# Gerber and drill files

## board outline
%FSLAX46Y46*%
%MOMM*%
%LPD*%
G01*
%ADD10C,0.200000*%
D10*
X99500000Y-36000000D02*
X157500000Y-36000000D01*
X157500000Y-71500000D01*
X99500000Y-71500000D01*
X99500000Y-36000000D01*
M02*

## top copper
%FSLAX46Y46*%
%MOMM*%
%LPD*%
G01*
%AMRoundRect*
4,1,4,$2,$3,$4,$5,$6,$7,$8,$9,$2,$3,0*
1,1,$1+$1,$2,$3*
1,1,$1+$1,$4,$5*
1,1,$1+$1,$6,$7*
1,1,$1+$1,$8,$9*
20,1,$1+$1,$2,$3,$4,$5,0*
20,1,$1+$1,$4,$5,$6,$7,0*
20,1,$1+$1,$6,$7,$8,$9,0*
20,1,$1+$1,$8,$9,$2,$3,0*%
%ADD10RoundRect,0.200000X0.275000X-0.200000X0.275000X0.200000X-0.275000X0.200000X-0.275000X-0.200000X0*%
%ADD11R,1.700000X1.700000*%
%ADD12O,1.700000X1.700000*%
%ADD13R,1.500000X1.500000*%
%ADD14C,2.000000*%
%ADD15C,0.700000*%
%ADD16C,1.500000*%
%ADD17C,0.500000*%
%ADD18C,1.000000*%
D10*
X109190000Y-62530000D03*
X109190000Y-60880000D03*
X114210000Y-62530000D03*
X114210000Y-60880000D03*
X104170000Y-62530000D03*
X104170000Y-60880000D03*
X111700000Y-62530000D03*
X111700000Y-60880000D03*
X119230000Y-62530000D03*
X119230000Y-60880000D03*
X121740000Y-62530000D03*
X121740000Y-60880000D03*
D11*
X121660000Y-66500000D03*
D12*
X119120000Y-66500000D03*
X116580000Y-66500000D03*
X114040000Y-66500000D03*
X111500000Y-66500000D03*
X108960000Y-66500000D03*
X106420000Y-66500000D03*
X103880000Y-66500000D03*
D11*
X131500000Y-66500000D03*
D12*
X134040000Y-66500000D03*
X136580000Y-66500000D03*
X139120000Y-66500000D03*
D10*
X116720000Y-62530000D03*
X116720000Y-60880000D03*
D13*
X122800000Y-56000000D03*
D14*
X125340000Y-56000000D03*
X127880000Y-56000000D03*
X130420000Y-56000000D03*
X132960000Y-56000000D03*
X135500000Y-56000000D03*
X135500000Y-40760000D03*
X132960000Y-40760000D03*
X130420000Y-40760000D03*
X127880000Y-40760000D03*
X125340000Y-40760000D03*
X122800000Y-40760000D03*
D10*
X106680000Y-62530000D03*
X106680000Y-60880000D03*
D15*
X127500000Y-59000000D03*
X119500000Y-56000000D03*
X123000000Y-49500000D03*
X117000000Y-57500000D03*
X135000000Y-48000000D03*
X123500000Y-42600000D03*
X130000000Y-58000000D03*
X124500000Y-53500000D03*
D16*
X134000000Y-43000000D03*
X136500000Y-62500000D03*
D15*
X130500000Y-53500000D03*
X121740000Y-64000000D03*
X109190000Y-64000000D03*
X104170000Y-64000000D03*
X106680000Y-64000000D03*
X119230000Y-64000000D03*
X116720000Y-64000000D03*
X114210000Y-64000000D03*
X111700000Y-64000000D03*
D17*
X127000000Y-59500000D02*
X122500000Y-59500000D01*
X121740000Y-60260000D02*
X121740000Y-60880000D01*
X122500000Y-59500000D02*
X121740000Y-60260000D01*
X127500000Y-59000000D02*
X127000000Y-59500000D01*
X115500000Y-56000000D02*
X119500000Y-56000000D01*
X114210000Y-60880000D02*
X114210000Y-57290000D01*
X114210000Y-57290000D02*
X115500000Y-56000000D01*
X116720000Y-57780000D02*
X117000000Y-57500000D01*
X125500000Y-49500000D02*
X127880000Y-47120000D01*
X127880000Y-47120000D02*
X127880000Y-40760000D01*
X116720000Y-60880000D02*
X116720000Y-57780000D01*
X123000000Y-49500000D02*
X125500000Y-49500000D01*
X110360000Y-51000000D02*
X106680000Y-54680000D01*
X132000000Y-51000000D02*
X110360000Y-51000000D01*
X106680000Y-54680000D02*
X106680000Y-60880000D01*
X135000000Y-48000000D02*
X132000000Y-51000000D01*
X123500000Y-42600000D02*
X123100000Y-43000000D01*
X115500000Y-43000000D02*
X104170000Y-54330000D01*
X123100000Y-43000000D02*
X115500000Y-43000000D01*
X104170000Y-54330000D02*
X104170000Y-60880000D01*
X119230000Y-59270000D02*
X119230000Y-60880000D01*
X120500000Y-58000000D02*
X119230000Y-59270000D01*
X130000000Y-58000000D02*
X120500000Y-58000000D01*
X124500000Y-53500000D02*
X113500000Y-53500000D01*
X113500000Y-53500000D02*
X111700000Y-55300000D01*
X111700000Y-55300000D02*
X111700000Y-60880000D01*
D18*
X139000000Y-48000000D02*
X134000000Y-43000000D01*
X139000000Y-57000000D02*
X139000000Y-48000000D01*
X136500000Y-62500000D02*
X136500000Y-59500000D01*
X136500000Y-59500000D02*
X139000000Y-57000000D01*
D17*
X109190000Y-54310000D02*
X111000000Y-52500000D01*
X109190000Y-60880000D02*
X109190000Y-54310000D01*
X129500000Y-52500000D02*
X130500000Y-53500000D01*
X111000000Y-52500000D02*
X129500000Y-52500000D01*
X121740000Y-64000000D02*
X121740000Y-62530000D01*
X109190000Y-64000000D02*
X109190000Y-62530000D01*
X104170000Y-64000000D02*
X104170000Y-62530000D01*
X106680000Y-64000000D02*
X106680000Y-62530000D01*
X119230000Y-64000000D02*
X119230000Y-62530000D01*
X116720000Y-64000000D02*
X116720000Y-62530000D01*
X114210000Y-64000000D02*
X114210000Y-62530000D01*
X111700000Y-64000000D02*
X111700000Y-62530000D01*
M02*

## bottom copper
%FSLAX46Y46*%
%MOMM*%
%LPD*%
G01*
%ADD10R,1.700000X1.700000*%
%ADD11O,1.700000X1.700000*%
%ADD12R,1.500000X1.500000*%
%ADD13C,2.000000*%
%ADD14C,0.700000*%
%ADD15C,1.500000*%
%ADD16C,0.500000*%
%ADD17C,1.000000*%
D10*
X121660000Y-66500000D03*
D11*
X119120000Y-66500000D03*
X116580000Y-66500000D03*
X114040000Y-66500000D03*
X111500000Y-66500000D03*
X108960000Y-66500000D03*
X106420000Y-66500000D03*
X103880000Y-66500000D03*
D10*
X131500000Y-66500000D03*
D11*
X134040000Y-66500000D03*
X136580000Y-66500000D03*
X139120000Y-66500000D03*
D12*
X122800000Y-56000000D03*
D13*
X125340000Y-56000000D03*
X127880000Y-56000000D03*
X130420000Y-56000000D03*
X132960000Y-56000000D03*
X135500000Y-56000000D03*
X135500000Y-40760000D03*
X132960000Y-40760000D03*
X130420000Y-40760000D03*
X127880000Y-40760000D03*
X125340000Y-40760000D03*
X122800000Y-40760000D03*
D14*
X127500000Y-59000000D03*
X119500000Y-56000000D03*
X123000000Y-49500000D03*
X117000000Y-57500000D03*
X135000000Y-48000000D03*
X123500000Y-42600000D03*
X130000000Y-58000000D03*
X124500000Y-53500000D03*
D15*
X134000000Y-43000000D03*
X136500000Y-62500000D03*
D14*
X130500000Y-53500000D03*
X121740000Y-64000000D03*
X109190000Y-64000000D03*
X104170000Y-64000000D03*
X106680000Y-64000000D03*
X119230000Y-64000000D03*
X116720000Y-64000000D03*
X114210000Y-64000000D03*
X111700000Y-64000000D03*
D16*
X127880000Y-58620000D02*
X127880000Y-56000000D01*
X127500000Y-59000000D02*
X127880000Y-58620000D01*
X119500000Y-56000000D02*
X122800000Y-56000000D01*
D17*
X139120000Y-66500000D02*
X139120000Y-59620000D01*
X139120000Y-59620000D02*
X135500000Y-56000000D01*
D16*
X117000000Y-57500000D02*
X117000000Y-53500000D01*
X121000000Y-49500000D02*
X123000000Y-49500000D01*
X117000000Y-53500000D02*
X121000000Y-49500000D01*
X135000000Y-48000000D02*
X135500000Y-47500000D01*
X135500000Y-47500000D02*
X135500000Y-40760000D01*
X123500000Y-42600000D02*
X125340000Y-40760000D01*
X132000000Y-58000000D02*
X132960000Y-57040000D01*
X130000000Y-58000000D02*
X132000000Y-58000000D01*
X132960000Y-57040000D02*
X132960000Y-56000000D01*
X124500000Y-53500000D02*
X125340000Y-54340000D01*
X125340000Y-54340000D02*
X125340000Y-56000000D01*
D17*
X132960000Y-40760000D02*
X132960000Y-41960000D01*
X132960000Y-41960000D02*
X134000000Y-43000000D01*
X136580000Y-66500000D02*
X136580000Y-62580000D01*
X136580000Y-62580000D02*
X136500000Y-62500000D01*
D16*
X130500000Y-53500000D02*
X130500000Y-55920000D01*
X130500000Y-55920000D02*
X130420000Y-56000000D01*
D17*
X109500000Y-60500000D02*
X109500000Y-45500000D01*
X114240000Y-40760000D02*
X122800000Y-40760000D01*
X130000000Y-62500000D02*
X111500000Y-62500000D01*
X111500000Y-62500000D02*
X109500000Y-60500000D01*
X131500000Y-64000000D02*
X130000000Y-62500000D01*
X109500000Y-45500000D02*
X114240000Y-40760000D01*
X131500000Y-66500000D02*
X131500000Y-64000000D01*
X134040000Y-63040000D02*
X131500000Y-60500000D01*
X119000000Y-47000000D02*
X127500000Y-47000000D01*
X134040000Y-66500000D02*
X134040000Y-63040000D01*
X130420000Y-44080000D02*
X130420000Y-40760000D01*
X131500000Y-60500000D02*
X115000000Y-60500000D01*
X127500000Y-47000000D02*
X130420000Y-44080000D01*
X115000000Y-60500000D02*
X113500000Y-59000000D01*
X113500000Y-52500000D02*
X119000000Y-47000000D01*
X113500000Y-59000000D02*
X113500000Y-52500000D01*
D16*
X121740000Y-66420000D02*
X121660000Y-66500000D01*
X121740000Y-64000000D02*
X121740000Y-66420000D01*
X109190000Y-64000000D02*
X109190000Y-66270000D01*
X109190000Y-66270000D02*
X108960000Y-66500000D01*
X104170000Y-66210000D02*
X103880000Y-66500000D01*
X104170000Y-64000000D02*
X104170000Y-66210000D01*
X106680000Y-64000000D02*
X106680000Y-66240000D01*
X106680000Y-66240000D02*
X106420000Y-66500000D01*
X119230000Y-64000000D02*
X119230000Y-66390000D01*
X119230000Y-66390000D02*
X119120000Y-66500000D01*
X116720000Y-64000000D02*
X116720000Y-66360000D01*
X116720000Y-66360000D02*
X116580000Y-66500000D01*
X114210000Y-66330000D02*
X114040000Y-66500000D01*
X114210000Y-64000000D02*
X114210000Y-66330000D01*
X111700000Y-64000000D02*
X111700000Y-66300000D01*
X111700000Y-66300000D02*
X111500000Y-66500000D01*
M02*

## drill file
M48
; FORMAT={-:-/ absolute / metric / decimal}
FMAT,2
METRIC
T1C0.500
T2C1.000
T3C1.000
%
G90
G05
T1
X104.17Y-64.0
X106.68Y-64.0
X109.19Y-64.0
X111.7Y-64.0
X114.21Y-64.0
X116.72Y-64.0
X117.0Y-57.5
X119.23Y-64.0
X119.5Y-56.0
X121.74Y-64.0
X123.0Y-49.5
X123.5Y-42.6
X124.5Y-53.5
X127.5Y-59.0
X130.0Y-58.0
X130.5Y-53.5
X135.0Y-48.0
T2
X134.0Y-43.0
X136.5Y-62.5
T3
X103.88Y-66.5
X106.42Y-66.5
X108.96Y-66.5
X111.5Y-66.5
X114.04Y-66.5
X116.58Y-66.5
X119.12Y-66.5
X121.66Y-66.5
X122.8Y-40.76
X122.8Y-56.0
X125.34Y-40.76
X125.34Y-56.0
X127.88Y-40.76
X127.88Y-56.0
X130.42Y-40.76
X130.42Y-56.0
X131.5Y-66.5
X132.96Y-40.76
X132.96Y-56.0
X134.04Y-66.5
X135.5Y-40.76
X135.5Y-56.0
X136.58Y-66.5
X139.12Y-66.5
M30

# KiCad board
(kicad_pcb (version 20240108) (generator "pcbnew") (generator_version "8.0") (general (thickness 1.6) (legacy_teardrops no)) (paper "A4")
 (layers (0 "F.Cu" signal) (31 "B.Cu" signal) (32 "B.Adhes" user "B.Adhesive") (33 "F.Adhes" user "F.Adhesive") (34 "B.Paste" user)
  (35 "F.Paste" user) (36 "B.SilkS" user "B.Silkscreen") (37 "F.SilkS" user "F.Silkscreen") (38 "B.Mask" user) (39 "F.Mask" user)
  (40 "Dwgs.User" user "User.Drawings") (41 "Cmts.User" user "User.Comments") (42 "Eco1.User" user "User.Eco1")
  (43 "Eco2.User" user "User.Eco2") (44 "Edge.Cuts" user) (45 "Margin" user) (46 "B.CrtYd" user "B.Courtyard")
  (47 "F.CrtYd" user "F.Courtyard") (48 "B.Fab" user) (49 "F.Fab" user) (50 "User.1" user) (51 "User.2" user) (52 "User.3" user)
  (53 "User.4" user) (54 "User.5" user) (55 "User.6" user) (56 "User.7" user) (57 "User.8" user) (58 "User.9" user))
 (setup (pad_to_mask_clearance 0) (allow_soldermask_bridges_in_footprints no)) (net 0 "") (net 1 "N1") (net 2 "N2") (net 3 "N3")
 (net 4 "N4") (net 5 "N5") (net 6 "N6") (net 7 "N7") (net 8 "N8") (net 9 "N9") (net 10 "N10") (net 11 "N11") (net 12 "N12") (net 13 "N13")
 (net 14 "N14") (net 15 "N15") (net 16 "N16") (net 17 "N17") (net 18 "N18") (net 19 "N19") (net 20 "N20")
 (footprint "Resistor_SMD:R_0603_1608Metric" (layer "F.Cu") (at 109.19 61.705 90)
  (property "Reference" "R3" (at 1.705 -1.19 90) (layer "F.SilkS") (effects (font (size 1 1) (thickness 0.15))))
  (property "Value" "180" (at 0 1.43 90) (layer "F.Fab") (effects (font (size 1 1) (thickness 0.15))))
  (pad "1" smd roundrect (at -0.825 0 90) (size 0.8 0.95) (layers "F.Cu" "F.Paste" "F.Mask") (roundrect_rratio 0.25) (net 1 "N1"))
  (pad "2" smd roundrect (at 0.825 0 90) (size 0.8 0.95) (layers "F.Cu" "F.Paste" "F.Mask") (roundrect_rratio 0.25) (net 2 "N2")))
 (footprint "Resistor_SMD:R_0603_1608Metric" (layer "F.Cu") (at 114.21 61.705 90)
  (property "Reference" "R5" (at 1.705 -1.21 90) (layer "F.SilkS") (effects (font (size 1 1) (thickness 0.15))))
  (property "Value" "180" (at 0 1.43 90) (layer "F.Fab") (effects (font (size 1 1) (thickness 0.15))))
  (pad "1" smd roundrect (at -0.825 0 90) (size 0.8 0.95) (layers "F.Cu" "F.Paste" "F.Mask") (roundrect_rratio 0.25) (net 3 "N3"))
  (pad "2" smd roundrect (at 0.825 0 90) (size 0.8 0.95) (layers "F.Cu" "F.Paste" "F.Mask") (roundrect_rratio 0.25) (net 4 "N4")))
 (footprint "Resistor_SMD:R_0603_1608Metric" (layer "F.Cu") (at 104.17 61.705 90)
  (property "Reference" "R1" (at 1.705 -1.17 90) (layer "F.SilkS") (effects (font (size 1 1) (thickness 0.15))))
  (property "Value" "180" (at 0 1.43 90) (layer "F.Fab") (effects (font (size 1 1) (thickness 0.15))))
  (pad "1" smd roundrect (at -0.825 0 90) (size 0.8 0.95) (layers "F.Cu" "F.Paste" "F.Mask") (roundrect_rratio 0.25) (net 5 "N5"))
  (pad "2" smd roundrect (at 0.825 0 90) (size 0.8 0.95) (layers "F.Cu" "F.Paste" "F.Mask") (roundrect_rratio 0.25) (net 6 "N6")))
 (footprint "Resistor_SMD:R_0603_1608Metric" (layer "F.Cu") (at 111.7 61.705 90)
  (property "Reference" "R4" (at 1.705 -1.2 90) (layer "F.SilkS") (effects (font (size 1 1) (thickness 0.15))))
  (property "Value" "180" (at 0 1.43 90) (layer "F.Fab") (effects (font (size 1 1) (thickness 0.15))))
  (pad "1" smd roundrect (at -0.825 0 90) (size 0.8 0.95) (layers "F.Cu" "F.Paste" "F.Mask") (roundrect_rratio 0.25) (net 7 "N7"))
  (pad "2" smd roundrect (at 0.825 0 90) (size 0.8 0.95) (layers "F.Cu" "F.Paste" "F.Mask") (roundrect_rratio 0.25) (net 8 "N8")))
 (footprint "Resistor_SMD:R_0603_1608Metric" (layer "F.Cu") (at 119.23 61.705 90)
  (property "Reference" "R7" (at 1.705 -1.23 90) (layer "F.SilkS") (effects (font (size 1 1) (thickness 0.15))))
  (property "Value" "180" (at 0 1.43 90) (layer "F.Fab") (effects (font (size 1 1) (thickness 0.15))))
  (pad "1" smd roundrect (at -0.825 0 90) (size 0.8 0.95) (layers "F.Cu" "F.Paste" "F.Mask") (roundrect_rratio 0.25) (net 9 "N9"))
  (pad "2" smd roundrect (at 0.825 0 90) (size 0.8 0.95) (layers "F.Cu" "F.Paste" "F.Mask") (roundrect_rratio 0.25) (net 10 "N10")))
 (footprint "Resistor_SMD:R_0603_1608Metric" (layer "F.Cu") (at 121.74 61.705 90)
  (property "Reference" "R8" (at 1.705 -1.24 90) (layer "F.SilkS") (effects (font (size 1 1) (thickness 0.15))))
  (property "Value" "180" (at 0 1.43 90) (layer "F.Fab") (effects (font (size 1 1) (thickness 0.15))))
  (pad "1" smd roundrect (at -0.825 0 90) (size 0.8 0.95) (layers "F.Cu" "F.Paste" "F.Mask") (roundrect_rratio 0.25) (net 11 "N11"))
  (pad "2" smd roundrect (at 0.825 0 90) (size 0.8 0.95) (layers "F.Cu" "F.Paste" "F.Mask") (roundrect_rratio 0.25) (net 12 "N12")))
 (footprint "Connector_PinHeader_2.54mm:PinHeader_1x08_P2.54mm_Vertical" (layer "F.Cu") (at 121.66 66.5 -90)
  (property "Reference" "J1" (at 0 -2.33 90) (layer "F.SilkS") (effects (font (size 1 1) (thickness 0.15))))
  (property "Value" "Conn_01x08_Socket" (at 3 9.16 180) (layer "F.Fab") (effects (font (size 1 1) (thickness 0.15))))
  (pad "1" thru_hole rect (at 0 0 270) (size 1.7 1.7) (drill 1) (layers "*.Cu" "*.Mask") (remove_unused_layers no) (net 11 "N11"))
  (pad "2" thru_hole oval (at 0 2.54 270) (size 1.7 1.7) (drill 1) (layers "*.Cu" "*.Mask") (remove_unused_layers no) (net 9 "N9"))
  (pad "3" thru_hole oval (at 0 5.08 270) (size 1.7 1.7) (drill 1) (layers "*.Cu" "*.Mask") (remove_unused_layers no) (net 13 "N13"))
  (pad "4" thru_hole oval (at 0 7.62 270) (size 1.7 1.7) (drill 1) (layers "*.Cu" "*.Mask") (remove_unused_layers no) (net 3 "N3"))
  (pad "5" thru_hole oval (at 0 10.16 270) (size 1.7 1.7) (drill 1) (layers "*.Cu" "*.Mask") (remove_unused_layers no) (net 7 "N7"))
  (pad "6" thru_hole oval (at 0 12.7 270) (size 1.7 1.7) (drill 1) (layers "*.Cu" "*.Mask") (remove_unused_layers no) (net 1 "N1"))
  (pad "7" thru_hole oval (at 0 15.24 270) (size 1.7 1.7) (drill 1) (layers "*.Cu" "*.Mask") (remove_unused_layers no) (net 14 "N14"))
  (pad "8" thru_hole oval (at 0 17.78 270) (size 1.7 1.7) (drill 1) (layers "*.Cu" "*.Mask") (remove_unused_layers no) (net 5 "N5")))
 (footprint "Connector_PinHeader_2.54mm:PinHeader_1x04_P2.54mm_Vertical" (layer "F.Cu") (at 131.5 66.5 90)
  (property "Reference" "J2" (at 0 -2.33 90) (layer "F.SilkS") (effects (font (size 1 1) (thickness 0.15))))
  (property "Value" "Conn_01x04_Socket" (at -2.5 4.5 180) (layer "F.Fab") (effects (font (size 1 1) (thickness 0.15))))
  (pad "1" thru_hole rect (at 0 0 90) (size 1.7 1.7) (drill 1) (layers "*.Cu" "*.Mask") (remove_unused_layers no) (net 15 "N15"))
  (pad "2" thru_hole oval (at 0 2.54 90) (size 1.7 1.7) (drill 1) (layers "*.Cu" "*.Mask") (remove_unused_layers no) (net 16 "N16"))
  (pad "3" thru_hole oval (at 0 5.08 90) (size 1.7 1.7) (drill 1) (layers "*.Cu" "*.Mask") (remove_unused_layers no) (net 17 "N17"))
  (pad "4" thru_hole oval (at 0 7.62 90) (size 1.7 1.7) (drill 1) (layers "*.Cu" "*.Mask") (remove_unused_layers no) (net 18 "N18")))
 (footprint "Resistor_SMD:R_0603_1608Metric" (layer "F.Cu") (at 116.72 61.705 90)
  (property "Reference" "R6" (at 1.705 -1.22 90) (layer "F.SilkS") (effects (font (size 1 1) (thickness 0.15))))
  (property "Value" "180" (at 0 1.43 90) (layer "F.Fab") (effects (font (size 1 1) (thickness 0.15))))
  (pad "1" smd roundrect (at -0.825 0 90) (size 0.8 0.95) (layers "F.Cu" "F.Paste" "F.Mask") (roundrect_rratio 0.25) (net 13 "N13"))
  (pad "2" smd roundrect (at 0.825 0 90) (size 0.8 0.95) (layers "F.Cu" "F.Paste" "F.Mask") (roundrect_rratio 0.25) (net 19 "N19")))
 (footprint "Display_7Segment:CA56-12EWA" (layer "F.Cu") (at 122.8 56 90)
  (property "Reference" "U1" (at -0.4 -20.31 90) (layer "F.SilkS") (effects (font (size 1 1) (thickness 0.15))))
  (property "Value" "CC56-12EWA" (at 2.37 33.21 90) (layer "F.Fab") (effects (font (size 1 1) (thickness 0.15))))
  (pad "1" thru_hole rect (at 0 0 90) (size 1.5 1.5) (drill 1) (layers "*.Cu" "*.Mask") (remove_unused_layers no) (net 4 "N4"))
  (pad "2" thru_hole circle (at 0 2.54 90) (size 2 2) (drill 1) (layers "*.Cu" "*.Mask") (remove_unused_layers no) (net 8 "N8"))
  (pad "3" thru_hole circle (at 0 5.08 90) (size 2 2) (drill 1) (layers "*.Cu" "*.Mask") (remove_unused_layers no) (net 12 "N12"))
  (pad "4" thru_hole circle (at 0 7.62 90) (size 2 2) (drill 1) (layers "*.Cu" "*.Mask") (remove_unused_layers no) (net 2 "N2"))
  (pad "5" thru_hole circle (at 0 10.16 90) (size 2 2) (drill 1) (layers "*.Cu" "*.Mask") (remove_unused_layers no) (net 10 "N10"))
  (pad "6" thru_hole circle (at 0 12.7 90) (size 2 2) (drill 1) (layers "*.Cu" "*.Mask") (remove_unused_layers no) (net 18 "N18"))
  (pad "7" thru_hole circle (at 15.24 12.7 90) (size 2 2) (drill 1) (layers "*.Cu" "*.Mask") (remove_unused_layers no) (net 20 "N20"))
  (pad "8" thru_hole circle (at 15.24 10.16 90) (size 2 2) (drill 1) (layers "*.Cu" "*.Mask") (remove_unused_layers no) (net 17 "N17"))
  (pad "9" thru_hole circle (at 15.24 7.62 90) (size 2 2) (drill 1) (layers "*.Cu" "*.Mask") (remove_unused_layers no) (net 16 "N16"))
  (pad "10" thru_hole circle (at 15.24 5.08 90) (size 2 2) (drill 1) (layers "*.Cu" "*.Mask") (remove_unused_layers no) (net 19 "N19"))
  (pad "11" thru_hole circle (at 15.24 2.54 90) (size 2 2) (drill 1) (layers "*.Cu" "*.Mask") (remove_unused_layers no) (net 6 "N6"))
  (pad "12" thru_hole circle (at 15.24 0 90) (size 2 2) (drill 1) (layers "*.Cu" "*.Mask") (remove_unused_layers no) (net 15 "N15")))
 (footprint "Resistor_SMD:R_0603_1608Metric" (layer "F.Cu") (at 106.68 61.705 90)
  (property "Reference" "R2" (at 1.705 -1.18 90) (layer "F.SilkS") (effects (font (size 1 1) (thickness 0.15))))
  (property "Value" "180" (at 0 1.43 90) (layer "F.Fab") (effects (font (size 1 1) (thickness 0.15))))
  (pad "1" smd roundrect (at -0.825 0 90) (size 0.8 0.95) (layers "F.Cu" "F.Paste" "F.Mask") (roundrect_rratio 0.25) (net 14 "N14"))
  (pad "2" smd roundrect (at 0.825 0 90) (size 0.8 0.95) (layers "F.Cu" "F.Paste" "F.Mask") (roundrect_rratio 0.25) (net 20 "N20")))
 (gr_rect (start 99.5 36) (end 157.5 71.5) (stroke (width 0.2) (type default)) (fill none) (layer "Edge.Cuts"))
 (segment (start 127 59.5) (end 122.5 59.5) (width 0.5) (layer "F.Cu") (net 12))
 (segment (start 121.74 60.26) (end 121.74 60.88) (width 0.5) (layer "F.Cu") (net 12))
 (segment (start 122.5 59.5) (end 121.74 60.26) (width 0.5) (layer "F.Cu") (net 12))
 (segment (start 127.5 59) (end 127 59.5) (width 0.5) (layer "F.Cu") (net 12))
 (via (at 127.5 59) (size 0.7) (drill 0.5) (layers "F.Cu" "B.Cu") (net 12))
 (segment (start 127.88 58.62) (end 127.88 56) (width 0.5) (layer "B.Cu") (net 12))
 (segment (start 127.5 59) (end 127.88 58.62) (width 0.5) (layer "B.Cu") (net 12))
 (segment (start 115.5 56) (end 119.5 56) (width 0.5) (layer "F.Cu") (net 4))
 (segment (start 114.21 60.88) (end 114.21 57.29) (width 0.5) (layer "F.Cu") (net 4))
 (segment (start 114.21 57.29) (end 115.5 56) (width 0.5) (layer "F.Cu") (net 4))
 (via (at 119.5 56) (size 0.7) (drill 0.5) (layers "F.Cu" "B.Cu") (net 4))
 (segment (start 119.5 56) (end 122.8 56) (width 0.5) (layer "B.Cu") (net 4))
 (segment (start 139.12 66.5) (end 139.12 59.62) (width 1) (layer "B.Cu") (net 18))
 (segment (start 139.12 59.62) (end 135.5 56) (width 1) (layer "B.Cu") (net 18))
 (segment (start 116.72 57.78) (end 117 57.5) (width 0.5) (layer "F.Cu") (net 19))
 (segment (start 125.5 49.5) (end 127.88 47.12) (width 0.5) (layer "F.Cu") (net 19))
 (segment (start 127.88 47.12) (end 127.88 40.76) (width 0.5) (layer "F.Cu") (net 19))
 (segment (start 116.72 60.88) (end 116.72 57.78) (width 0.5) (layer "F.Cu") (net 19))
 (segment (start 123 49.5) (end 125.5 49.5) (width 0.5) (layer "F.Cu") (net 19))
 (via (at 123 49.5) (size 0.7) (drill 0.5) (layers "F.Cu" "B.Cu") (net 19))
 (via (at 117 57.5) (size 0.7) (drill 0.5) (layers "F.Cu" "B.Cu") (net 19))
 (segment (start 117 57.5) (end 117 53.5) (width 0.5) (layer "B.Cu") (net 19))
 (segment (start 121 49.5) (end 123 49.5) (width 0.5) (layer "B.Cu") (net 19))
 (segment (start 117 53.5) (end 121 49.5) (width 0.5) (layer "B.Cu") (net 19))
 (segment (start 110.36 51) (end 106.68 54.68) (width 0.5) (layer "F.Cu") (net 20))
 (segment (start 132 51) (end 110.36 51) (width 0.5) (layer "F.Cu") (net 20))
 (segment (start 106.68 54.68) (end 106.68 60.88) (width 0.5) (layer "F.Cu") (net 20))
 (segment (start 135 48) (end 132 51) (width 0.5) (layer "F.Cu") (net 20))
 (via (at 135 48) (size 0.7) (drill 0.5) (layers "F.Cu" "B.Cu") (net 20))
 (segment (start 135 48) (end 135.5 47.5) (width 0.5) (layer "B.Cu") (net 20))
 (segment (start 135.5 47.5) (end 135.5 40.76) (width 0.5) (layer "B.Cu") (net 20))
 (segment (start 123.5 42.6) (end 123.1 43) (width 0.5) (layer "F.Cu") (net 6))
 (segment (start 115.5 43) (end 104.17 54.33) (width 0.5) (layer "F.Cu") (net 6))
 (segment (start 123.1 43) (end 115.5 43) (width 0.5) (layer "F.Cu") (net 6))
 (segment (start 104.17 54.33) (end 104.17 60.88) (width 0.5) (layer "F.Cu") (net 6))
 (via (at 123.5 42.6) (size 0.7) (drill 0.5) (layers "F.Cu" "B.Cu") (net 6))
 (segment (start 123.5 42.6) (end 125.34 40.76) (width 0.5) (layer "B.Cu") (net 6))
 (segment (start 119.23 59.27) (end 119.23 60.88) (width 0.5) (layer "F.Cu") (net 10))
 (segment (start 120.5 58) (end 119.23 59.27) (width 0.5) (layer "F.Cu") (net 10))
 (segment (start 130 58) (end 120.5 58) (width 0.5) (layer "F.Cu") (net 10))
 (via (at 130 58) (size 0.7) (drill 0.5) (layers "F.Cu" "B.Cu") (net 10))
 (segment (start 132 58) (end 132.96 57.04) (width 0.5) (layer "B.Cu") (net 10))
 (segment (start 130 58) (end 132 58) (width 0.5) (layer "B.Cu") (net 10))
 (segment (start 132.96 57.04) (end 132.96 56) (width 0.5) (layer "B.Cu") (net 10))
 (segment (start 124.5 53.5) (end 113.5 53.5) (width 0.5) (layer "F.Cu") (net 8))
 (segment (start 113.5 53.5) (end 111.7 55.3) (width 0.5) (layer "F.Cu") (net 8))
 (segment (start 111.7 55.3) (end 111.7 60.88) (width 0.5) (layer "F.Cu") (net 8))
 (via (at 124.5 53.5) (size 0.7) (drill 0.5) (layers "F.Cu" "B.Cu") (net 8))
 (segment (start 124.5 53.5) (end 125.34 54.34) (width 0.5) (layer "B.Cu") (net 8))
 (segment (start 125.34 54.34) (end 125.34 56) (width 0.5) (layer "B.Cu") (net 8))
 (segment (start 139 48) (end 134 43) (width 1) (layer "F.Cu") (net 17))
 (segment (start 139 57) (end 139 48) (width 1) (layer "F.Cu") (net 17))
 (segment (start 136.5 62.5) (end 136.5 59.5) (width 1) (layer "F.Cu") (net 17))
 (segment (start 136.5 59.5) (end 139 57) (width 1) (layer "F.Cu") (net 17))
 (via (at 134 43) (size 1.5) (drill 1) (layers "F.Cu" "B.Cu") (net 17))
 (via (at 136.5 62.5) (size 1.5) (drill 1) (layers "F.Cu" "B.Cu") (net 17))
 (segment (start 132.96 40.76) (end 132.96 41.96) (width 1) (layer "B.Cu") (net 17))
 (segment (start 132.96 41.96) (end 134 43) (width 1) (layer "B.Cu") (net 17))
 (segment (start 136.58 66.5) (end 136.58 62.58) (width 1) (layer "B.Cu") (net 17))
 (segment (start 136.58 62.58) (end 136.5 62.5) (width 1) (layer "B.Cu") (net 17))
 (segment (start 109.19 54.31) (end 111 52.5) (width 0.5) (layer "F.Cu") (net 2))
 (segment (start 109.19 60.88) (end 109.19 54.31) (width 0.5) (layer "F.Cu") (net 2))
 (segment (start 129.5 52.5) (end 130.5 53.5) (width 0.5) (layer "F.Cu") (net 2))
 (segment (start 111 52.5) (end 129.5 52.5) (width 0.5) (layer "F.Cu") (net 2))
 (via (at 130.5 53.5) (size 0.7) (drill 0.5) (layers "F.Cu" "B.Cu") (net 2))
 (segment (start 130.5 53.5) (end 130.5 55.92) (width 0.5) (layer "B.Cu") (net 2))
 (segment (start 130.5 55.92) (end 130.42 56) (width 0.5) (layer "B.Cu") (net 2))
 (segment (start 109.5 60.5) (end 109.5 45.5) (width 1) (layer "B.Cu") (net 15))
 (segment (start 114.24 40.76) (end 122.8 40.76) (width 1) (layer "B.Cu") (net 15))
 (segment (start 130 62.5) (end 111.5 62.5) (width 1) (layer "B.Cu") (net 15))
 (segment (start 111.5 62.5) (end 109.5 60.5) (width 1) (layer "B.Cu") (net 15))
 (segment (start 131.5 64) (end 130 62.5) (width 1) (layer "B.Cu") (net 15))
 (segment (start 109.5 45.5) (end 114.24 40.76) (width 1) (layer "B.Cu") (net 15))
 (segment (start 131.5 66.5) (end 131.5 64) (width 1) (layer "B.Cu") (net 15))
 (segment (start 134.04 63.04) (end 131.5 60.5) (width 1) (layer "B.Cu") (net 16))
 (segment (start 119 47) (end 127.5 47) (width 1) (layer "B.Cu") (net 16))
 (segment (start 134.04 66.5) (end 134.04 63.04) (width 1) (layer "B.Cu") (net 16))
 (segment (start 130.42 44.08) (end 130.42 40.76) (width 1) (layer "B.Cu") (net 16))
 (segment (start 131.5 60.5) (end 115 60.5) (width 1) (layer "B.Cu") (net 16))
 (segment (start 127.5 47) (end 130.42 44.08) (width 1) (layer "B.Cu") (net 16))
 (segment (start 115 60.5) (end 113.5 59) (width 1) (layer "B.Cu") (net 16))
 (segment (start 113.5 52.5) (end 119 47) (width 1) (layer "B.Cu") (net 16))
 (segment (start 113.5 59) (end 113.5 52.5) (width 1) (layer "B.Cu") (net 16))
 (segment (start 121.74 64) (end 121.74 62.53) (width 0.5) (layer "F.Cu") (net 11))
 (via (at 121.74 64) (size 0.7) (drill 0.5) (layers "F.Cu" "B.Cu") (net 11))
 (segment (start 121.74 66.42) (end 121.66 66.5) (width 0.5) (layer "B.Cu") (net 11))
 (segment (start 121.74 64) (end 121.74 66.42) (width 0.5) (layer "B.Cu") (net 11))
 (segment (start 109.19 64) (end 109.19 62.53) (width 0.5) (layer "F.Cu") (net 1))
 (via (at 109.19 64) (size 0.7) (drill 0.5) (layers "F.Cu" "B.Cu") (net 1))
 (segment (start 109.19 64) (end 109.19 66.27) (width 0.5) (layer "B.Cu") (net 1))
 (segment (start 109.19 66.27) (end 108.96 66.5) (width 0.5) (layer "B.Cu") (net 1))
 (segment (start 104.17 64) (end 104.17 62.53) (width 0.5) (layer "F.Cu") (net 5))
 (via (at 104.17 64) (size 0.7) (drill 0.5) (layers "F.Cu" "B.Cu") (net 5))
 (segment (start 104.17 66.21) (end 103.88 66.5) (width 0.5) (layer "B.Cu") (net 5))
 (segment (start 104.17 64) (end 104.17 66.21) (width 0.5) (layer "B.Cu") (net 5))
 (segment (start 106.68 64) (end 106.68 62.53) (width 0.5) (layer "F.Cu") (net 14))
 (via (at 106.68 64) (size 0.7) (drill 0.5) (layers "F.Cu" "B.Cu") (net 14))
 (segment (start 106.68 64) (end 106.68 66.24) (width 0.5) (layer "B.Cu") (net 14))
 (segment (start 106.68 66.24) (end 106.42 66.5) (width 0.5) (layer "B.Cu") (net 14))
 (segment (start 119.23 64) (end 119.23 62.53) (width 0.5) (layer "F.Cu") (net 9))
 (via (at 119.23 64) (size 0.7) (drill 0.5) (layers "F.Cu" "B.Cu") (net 9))
 (segment (start 119.23 64) (end 119.23 66.39) (width 0.5) (layer "B.Cu") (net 9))
 (segment (start 119.23 66.39) (end 119.12 66.5) (width 0.5) (layer "B.Cu") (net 9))
 (segment (start 116.72 64) (end 116.72 62.53) (width 0.5) (layer "F.Cu") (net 13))
 (via (at 116.72 64) (size 0.7) (drill 0.5) (layers "F.Cu" "B.Cu") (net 13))
 (segment (start 116.72 64) (end 116.72 66.36) (width 0.5) (layer "B.Cu") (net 13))
 (segment (start 116.72 66.36) (end 116.58 66.5) (width 0.5) (layer "B.Cu") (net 13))
 (segment (start 114.21 64) (end 114.21 62.53) (width 0.5) (layer "F.Cu") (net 3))
 (via (at 114.21 64) (size 0.7) (drill 0.5) (layers "F.Cu" "B.Cu") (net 3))
 (segment (start 114.21 66.33) (end 114.04 66.5) (width 0.5) (layer "B.Cu") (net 3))
 (segment (start 114.21 64) (end 114.21 66.33) (width 0.5) (layer "B.Cu") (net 3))
 (segment (start 111.7 64) (end 111.7 62.53) (width 0.5) (layer "F.Cu") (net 7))
 (via (at 111.7 64) (size 0.7) (drill 0.5) (layers "F.Cu" "B.Cu") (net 7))
 (segment (start 111.7 64) (end 111.7 66.3) (width 0.5) (layer "B.Cu") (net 7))
 (segment (start 111.7 66.3) (end 111.5 66.5) (width 0.5) (layer "B.Cu") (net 7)))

